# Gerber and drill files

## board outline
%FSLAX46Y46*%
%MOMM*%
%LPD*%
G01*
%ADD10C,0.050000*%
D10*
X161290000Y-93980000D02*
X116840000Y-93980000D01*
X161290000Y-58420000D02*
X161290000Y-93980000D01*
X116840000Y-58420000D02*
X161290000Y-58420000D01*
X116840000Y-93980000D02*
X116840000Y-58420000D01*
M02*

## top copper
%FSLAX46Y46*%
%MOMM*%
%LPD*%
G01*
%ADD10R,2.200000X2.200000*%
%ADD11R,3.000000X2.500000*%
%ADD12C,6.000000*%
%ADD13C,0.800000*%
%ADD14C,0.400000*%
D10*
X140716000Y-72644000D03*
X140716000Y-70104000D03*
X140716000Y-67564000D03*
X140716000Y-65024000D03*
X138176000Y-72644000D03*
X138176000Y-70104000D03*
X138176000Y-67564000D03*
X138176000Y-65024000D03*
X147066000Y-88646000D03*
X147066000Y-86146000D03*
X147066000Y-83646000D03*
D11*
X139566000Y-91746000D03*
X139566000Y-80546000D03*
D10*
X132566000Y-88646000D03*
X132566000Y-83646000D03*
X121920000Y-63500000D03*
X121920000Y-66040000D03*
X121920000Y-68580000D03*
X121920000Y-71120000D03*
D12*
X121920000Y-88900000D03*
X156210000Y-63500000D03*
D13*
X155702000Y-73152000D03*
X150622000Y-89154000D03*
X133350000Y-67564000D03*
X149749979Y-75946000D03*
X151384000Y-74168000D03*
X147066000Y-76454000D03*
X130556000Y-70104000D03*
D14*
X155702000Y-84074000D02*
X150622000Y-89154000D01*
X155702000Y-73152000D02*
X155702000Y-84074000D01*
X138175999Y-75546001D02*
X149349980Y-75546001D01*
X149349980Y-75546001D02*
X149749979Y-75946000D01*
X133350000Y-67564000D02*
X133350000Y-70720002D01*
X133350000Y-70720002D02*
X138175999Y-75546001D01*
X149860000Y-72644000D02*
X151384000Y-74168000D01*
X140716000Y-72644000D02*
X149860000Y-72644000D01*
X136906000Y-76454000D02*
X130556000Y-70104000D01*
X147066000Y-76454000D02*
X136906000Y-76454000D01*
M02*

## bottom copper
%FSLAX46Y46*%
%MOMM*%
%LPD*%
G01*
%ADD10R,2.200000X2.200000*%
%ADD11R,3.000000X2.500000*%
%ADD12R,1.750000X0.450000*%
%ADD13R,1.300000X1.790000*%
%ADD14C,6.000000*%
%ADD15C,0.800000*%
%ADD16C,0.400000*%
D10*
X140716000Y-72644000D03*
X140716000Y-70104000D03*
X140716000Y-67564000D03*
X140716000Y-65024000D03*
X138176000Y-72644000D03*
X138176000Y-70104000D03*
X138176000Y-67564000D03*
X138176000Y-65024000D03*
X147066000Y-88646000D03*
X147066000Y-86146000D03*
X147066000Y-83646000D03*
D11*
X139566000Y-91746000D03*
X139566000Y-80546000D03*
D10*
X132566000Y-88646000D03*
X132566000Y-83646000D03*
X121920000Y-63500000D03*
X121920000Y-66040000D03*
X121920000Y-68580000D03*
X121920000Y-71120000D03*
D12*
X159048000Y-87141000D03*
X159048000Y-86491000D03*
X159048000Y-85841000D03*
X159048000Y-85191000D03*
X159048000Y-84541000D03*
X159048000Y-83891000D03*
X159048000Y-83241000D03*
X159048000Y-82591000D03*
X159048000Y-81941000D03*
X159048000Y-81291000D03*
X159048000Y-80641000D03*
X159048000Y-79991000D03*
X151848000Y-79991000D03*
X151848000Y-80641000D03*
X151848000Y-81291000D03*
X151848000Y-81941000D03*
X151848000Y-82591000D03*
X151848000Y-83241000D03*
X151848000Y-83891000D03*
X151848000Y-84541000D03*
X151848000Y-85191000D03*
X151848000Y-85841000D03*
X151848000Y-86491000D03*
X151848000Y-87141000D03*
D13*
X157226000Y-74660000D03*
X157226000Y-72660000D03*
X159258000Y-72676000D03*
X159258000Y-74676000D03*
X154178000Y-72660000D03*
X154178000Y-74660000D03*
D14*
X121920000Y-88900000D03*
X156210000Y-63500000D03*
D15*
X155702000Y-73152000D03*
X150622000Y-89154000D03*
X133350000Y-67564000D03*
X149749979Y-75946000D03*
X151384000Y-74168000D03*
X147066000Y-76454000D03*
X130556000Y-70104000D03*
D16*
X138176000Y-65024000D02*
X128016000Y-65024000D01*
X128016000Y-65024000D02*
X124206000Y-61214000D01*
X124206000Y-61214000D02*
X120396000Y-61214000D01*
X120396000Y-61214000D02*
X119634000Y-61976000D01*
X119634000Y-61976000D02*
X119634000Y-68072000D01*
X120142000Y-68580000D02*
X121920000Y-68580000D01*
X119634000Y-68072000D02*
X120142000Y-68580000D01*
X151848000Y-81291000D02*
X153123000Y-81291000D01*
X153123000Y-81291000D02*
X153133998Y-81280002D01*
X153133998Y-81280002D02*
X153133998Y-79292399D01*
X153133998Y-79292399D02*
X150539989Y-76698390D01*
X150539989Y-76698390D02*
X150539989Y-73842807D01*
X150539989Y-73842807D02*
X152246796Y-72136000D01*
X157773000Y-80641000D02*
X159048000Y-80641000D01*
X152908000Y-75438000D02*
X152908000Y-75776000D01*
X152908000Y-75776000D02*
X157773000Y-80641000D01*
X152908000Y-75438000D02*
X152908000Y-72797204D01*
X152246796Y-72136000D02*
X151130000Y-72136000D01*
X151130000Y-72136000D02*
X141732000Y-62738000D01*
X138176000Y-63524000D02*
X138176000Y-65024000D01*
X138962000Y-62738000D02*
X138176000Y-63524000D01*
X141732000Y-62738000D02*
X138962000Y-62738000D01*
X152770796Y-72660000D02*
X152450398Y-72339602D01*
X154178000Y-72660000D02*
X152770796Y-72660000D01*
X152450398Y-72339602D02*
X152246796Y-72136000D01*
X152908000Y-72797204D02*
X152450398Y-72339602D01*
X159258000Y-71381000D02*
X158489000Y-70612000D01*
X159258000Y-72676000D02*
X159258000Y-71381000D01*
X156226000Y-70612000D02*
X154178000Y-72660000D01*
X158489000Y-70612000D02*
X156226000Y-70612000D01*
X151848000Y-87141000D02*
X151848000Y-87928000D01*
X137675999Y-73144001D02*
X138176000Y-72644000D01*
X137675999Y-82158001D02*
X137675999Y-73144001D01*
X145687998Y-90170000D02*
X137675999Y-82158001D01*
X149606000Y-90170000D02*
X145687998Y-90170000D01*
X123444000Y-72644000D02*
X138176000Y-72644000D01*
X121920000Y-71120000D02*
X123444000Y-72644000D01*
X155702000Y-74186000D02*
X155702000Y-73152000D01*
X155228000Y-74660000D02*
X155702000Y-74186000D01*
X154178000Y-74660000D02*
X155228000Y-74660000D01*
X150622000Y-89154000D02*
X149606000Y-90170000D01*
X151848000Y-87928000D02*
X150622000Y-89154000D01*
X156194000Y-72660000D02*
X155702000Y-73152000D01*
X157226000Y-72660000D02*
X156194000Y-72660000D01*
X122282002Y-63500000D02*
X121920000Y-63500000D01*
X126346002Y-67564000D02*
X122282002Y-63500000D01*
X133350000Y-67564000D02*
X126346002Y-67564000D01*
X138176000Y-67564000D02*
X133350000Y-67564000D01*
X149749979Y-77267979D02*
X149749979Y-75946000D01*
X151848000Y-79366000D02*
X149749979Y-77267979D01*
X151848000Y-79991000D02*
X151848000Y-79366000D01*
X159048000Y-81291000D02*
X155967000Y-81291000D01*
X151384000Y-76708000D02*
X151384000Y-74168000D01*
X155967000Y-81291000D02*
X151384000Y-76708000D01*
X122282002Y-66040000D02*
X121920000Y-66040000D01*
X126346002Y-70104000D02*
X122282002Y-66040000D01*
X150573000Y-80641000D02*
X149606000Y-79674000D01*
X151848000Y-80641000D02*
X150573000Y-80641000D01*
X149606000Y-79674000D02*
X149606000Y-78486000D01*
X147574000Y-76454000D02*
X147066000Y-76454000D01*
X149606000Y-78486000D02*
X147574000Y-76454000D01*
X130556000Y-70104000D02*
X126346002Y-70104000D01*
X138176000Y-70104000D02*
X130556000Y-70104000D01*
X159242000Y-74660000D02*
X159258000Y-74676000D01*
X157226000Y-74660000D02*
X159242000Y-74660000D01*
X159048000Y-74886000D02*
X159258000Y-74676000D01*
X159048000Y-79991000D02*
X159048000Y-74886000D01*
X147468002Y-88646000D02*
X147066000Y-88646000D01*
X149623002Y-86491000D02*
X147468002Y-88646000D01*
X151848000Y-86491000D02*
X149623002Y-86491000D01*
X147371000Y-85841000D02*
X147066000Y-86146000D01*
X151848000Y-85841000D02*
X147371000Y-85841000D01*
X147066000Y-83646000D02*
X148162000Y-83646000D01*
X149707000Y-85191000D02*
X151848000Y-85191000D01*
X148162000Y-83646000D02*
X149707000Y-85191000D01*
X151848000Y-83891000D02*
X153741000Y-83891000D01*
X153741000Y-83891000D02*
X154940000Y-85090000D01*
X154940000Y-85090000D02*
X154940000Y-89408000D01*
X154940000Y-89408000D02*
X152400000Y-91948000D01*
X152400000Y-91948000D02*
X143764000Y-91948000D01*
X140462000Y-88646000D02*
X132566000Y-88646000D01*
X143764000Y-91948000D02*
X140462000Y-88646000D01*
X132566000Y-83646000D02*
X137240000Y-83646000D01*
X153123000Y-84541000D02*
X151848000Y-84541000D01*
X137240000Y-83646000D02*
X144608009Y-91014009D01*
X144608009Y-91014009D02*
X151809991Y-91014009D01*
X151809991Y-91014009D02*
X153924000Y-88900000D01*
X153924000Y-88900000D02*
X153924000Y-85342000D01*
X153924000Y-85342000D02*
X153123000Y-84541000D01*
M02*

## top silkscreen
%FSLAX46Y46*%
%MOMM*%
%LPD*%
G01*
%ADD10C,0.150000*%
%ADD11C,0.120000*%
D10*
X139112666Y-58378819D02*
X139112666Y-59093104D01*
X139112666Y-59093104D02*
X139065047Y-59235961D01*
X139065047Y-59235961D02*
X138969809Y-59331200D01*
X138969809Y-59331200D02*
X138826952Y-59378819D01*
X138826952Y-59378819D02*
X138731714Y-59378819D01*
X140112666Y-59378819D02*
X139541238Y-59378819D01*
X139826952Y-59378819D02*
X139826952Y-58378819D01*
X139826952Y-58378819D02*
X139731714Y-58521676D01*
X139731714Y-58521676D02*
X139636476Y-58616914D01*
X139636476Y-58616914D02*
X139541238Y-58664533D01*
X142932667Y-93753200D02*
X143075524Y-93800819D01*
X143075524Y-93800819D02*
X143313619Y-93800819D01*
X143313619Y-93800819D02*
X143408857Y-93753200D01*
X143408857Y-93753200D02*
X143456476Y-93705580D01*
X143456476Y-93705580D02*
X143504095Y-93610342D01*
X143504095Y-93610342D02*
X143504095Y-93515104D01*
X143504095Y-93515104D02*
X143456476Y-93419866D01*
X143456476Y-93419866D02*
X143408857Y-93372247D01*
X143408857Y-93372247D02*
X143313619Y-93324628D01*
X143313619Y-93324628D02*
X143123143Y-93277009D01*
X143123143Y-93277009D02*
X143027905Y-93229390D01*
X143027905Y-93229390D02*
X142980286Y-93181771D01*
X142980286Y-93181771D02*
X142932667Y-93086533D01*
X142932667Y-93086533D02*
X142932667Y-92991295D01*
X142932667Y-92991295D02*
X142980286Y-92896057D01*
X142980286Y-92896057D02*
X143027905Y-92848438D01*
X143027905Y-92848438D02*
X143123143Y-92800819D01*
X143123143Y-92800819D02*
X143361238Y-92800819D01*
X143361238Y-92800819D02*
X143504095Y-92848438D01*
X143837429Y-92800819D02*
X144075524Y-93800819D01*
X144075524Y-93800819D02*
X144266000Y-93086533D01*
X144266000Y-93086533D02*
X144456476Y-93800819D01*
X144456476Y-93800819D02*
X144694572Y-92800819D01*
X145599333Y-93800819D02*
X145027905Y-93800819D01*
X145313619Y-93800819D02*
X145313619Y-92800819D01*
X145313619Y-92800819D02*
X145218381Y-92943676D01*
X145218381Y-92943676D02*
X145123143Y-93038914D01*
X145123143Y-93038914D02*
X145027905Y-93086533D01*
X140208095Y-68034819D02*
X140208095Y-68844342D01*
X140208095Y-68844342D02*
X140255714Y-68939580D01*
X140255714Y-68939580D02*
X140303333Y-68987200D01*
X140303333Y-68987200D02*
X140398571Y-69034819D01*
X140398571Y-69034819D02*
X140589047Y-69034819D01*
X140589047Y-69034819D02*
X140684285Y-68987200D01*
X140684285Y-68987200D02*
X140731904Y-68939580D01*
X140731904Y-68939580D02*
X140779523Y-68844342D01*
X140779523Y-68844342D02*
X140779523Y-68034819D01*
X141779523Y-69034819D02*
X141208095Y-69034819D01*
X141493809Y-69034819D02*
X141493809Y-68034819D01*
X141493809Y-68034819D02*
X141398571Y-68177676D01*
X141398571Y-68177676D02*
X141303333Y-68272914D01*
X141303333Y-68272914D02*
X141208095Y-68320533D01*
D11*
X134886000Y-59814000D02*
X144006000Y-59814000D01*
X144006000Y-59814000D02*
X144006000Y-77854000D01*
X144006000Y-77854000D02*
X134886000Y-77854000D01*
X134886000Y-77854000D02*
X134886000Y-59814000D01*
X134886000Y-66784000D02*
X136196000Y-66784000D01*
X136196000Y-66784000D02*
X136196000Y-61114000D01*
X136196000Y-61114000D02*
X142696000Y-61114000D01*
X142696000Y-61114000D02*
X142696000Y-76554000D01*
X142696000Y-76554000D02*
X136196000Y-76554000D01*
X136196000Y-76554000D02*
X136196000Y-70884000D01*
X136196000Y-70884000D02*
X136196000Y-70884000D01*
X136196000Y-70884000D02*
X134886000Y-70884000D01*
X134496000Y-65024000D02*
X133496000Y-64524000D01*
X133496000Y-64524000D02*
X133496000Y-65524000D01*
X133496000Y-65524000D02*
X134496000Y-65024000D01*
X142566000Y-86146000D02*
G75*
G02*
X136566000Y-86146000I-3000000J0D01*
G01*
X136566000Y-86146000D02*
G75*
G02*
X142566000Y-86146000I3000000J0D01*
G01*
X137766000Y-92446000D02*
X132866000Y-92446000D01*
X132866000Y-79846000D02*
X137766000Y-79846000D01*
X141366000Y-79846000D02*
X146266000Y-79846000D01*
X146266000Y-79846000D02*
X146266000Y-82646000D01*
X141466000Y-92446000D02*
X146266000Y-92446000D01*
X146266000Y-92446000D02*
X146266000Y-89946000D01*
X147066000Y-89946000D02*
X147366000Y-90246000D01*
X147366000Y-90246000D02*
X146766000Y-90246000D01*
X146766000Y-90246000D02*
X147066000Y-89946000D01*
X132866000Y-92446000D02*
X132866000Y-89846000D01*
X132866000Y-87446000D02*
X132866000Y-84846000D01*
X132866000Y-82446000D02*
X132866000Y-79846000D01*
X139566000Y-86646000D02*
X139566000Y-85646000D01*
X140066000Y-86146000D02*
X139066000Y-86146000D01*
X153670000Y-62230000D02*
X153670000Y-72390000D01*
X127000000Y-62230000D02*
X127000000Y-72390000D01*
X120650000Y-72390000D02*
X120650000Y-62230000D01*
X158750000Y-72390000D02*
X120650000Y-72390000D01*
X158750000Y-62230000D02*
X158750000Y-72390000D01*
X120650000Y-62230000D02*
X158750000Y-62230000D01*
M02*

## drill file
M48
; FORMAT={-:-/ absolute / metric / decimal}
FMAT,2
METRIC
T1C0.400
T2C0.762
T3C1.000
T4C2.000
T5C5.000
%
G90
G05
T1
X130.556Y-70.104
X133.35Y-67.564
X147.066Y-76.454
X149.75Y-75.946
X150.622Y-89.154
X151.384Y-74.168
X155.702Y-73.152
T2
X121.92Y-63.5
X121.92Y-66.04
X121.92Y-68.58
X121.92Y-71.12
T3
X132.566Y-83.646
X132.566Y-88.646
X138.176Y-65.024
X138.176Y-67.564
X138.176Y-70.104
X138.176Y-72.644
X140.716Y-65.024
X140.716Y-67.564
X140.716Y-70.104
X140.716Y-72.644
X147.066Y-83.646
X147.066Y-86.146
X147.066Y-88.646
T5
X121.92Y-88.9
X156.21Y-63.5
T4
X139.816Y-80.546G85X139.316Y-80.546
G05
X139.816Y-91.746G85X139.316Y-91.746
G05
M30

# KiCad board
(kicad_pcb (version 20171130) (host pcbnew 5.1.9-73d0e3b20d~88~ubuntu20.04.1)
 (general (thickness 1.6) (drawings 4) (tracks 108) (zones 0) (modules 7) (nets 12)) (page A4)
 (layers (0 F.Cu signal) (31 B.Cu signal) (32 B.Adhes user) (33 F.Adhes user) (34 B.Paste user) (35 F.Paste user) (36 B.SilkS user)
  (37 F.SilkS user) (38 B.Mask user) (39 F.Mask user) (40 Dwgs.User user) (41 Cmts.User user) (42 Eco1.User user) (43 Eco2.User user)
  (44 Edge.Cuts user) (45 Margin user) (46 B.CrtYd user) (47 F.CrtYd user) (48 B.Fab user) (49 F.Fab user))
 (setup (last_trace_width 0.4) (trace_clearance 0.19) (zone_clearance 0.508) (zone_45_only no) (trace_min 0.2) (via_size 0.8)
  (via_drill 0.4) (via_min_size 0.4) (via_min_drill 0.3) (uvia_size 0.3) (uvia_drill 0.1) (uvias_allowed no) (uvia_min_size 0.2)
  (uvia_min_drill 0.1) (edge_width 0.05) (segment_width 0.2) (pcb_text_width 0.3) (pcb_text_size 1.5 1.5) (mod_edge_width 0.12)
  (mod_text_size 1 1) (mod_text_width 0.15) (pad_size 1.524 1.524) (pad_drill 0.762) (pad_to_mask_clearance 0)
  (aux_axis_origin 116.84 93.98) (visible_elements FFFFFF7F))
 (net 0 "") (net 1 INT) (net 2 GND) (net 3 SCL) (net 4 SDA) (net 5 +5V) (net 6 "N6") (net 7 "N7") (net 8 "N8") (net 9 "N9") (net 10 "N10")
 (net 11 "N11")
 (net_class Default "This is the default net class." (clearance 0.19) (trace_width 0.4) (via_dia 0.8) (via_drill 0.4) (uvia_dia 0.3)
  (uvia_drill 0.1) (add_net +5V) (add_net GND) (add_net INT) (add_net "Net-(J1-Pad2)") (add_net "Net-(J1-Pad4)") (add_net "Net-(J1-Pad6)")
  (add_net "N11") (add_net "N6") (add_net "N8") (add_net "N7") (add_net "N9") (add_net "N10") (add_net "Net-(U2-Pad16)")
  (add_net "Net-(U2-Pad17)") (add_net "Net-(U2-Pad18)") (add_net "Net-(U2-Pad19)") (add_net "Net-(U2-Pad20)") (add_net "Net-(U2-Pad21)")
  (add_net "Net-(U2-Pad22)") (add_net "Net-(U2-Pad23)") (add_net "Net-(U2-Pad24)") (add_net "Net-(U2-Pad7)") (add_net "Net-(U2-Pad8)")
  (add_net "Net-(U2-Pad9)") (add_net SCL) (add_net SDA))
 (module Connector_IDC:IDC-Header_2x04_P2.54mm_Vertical (layer F.Cu) (at 138.176 65.024)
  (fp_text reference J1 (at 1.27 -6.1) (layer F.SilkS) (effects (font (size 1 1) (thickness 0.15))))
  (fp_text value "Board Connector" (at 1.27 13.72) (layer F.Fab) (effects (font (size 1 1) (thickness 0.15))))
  (fp_line (start -3.29 -5.21) (end 5.83 -5.21) (layer F.SilkS) (width 0.12))
  (fp_line (start 5.83 -5.21) (end 5.83 12.83) (layer F.SilkS) (width 0.12))
  (fp_line (start 5.83 12.83) (end -3.29 12.83) (layer F.SilkS) (width 0.12))
  (fp_line (start -3.29 12.83) (end -3.29 -5.21) (layer F.SilkS) (width 0.12))
  (fp_line (start -3.29 1.76) (end -1.98 1.76) (layer F.SilkS) (width 0.12))
  (fp_line (start -1.98 1.76) (end -1.98 -3.91) (layer F.SilkS) (width 0.12))
  (fp_line (start -1.98 -3.91) (end 4.52 -3.91) (layer F.SilkS) (width 0.12))
  (fp_line (start 4.52 -3.91) (end 4.52 11.53) (layer F.SilkS) (width 0.12))
  (fp_line (start 4.52 11.53) (end -1.98 11.53) (layer F.SilkS) (width 0.12))
  (fp_line (start -1.98 11.53) (end -1.98 5.86) (layer F.SilkS) (width 0.12))
  (fp_line (start -1.98 5.86) (end -1.98 5.86) (layer F.SilkS) (width 0.12))
  (fp_line (start -1.98 5.86) (end -3.29 5.86) (layer F.SilkS) (width 0.12))
  (fp_line (start -3.68 0) (end -4.68 -0.5) (layer F.SilkS) (width 0.12))
  (fp_line (start -4.68 -0.5) (end -4.68 0.5) (layer F.SilkS) (width 0.12))
  (fp_line (start -4.68 0.5) (end -3.68 0) (layer F.SilkS) (width 0.12))
  (pad 8 thru_hole rect (at 2.54 7.62) (size 2.2 2.2) (drill 1) (layers *.Cu *.Mask) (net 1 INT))
  (pad 6 thru_hole rect (at 2.54 5.08) (size 2.2 2.2) (drill 1) (layers *.Cu *.Mask))
  (pad 4 thru_hole rect (at 2.54 2.54) (size 2.2 2.2) (drill 1) (layers *.Cu *.Mask))
  (pad 2 thru_hole rect (at 2.54 0) (size 2.2 2.2) (drill 1) (layers *.Cu *.Mask))
  (pad 7 thru_hole rect (at 0 7.62) (size 2.2 2.2) (drill 1) (layers *.Cu *.Mask) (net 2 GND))
  (pad 5 thru_hole rect (at 0 5.08) (size 2.2 2.2) (drill 1) (layers *.Cu *.Mask) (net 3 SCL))
  (pad 3 thru_hole rect (at 0 2.54) (size 2.2 2.2) (drill 1) (layers *.Cu *.Mask) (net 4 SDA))
  (pad 1 thru_hole rect (at 0 0) (size 2.2 2.2) (drill 1) (layers *.Cu *.Mask) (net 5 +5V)))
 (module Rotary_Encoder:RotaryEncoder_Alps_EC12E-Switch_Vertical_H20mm (layer F.Cu) (at 147.066 88.646 180)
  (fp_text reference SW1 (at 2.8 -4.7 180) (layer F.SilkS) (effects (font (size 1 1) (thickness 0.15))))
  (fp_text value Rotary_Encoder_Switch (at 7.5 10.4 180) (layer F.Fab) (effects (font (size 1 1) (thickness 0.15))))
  (fp_circle (center 7.5 2.5) (end 10.5 2.5) (layer F.SilkS) (width 0.12))
  (fp_line (start 9.3 -3.8) (end 14.2 -3.8) (layer F.SilkS) (width 0.12))
  (fp_line (start 14.2 8.8) (end 9.3 8.8) (layer F.SilkS) (width 0.12))
  (fp_line (start 5.7 8.8) (end 0.8 8.8) (layer F.SilkS) (width 0.12))
  (fp_line (start 0.8 8.8) (end 0.8 6) (layer F.SilkS) (width 0.12))
  (fp_line (start 5.6 -3.8) (end 0.8 -3.8) (layer F.SilkS) (width 0.12))
  (fp_line (start 0.8 -3.8) (end 0.8 -1.3) (layer F.SilkS) (width 0.12))
  (fp_line (start 0 -1.3) (end -0.3 -1.6) (layer F.SilkS) (width 0.12))
  (fp_line (start -0.3 -1.6) (end 0.3 -1.6) (layer F.SilkS) (width 0.12))
  (fp_line (start 0.3 -1.6) (end 0 -1.3) (layer F.SilkS) (width 0.12))
  (fp_line (start 14.2 -3.8) (end 14.2 -1.2) (layer F.SilkS) (width 0.12))
  (fp_line (start 14.2 1.2) (end 14.2 3.8) (layer F.SilkS) (width 0.12))
  (fp_line (start 14.2 6.2) (end 14.2 8.8) (layer F.SilkS) (width 0.12))
  (fp_line (start 7.5 2) (end 7.5 3) (layer F.SilkS) (width 0.12))
  (fp_line (start 7 2.5) (end 8 2.5) (layer F.SilkS) (width 0.12))
  (pad A thru_hole rect (at 0 0 180) (size 2.2 2.2) (drill 1) (layers *.Cu *.Mask) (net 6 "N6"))
  (pad C thru_hole rect (at 0 2.5 180) (size 2.2 2.2) (drill 1) (layers *.Cu *.Mask) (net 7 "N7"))
  (pad B thru_hole rect (at 0 5 180) (size 2.2 2.2) (drill 1) (layers *.Cu *.Mask) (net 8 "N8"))
  (pad MP thru_hole rect (at 7.5 -3.1 180) (size 3 2.5) (drill oval 2.5 2) (layers *.Cu *.Mask))
  (pad MP thru_hole rect (at 7.5 8.1 180) (size 3 2.5) (drill oval 2.5 2) (layers *.Cu *.Mask))
  (pad S1 thru_hole rect (at 14.5 0 180) (size 2.2 2.2) (drill 1) (layers *.Cu *.Mask) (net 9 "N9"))
  (pad S2 thru_hole rect (at 14.5 5 180) (size 2.2 2.2) (drill 1) (layers *.Cu *.Mask) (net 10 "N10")))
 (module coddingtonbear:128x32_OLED (layer F.Cu) (at 129.54 68.58)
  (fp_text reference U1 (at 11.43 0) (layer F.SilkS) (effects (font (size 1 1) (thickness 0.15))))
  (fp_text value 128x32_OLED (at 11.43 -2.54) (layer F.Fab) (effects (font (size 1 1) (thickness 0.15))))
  (fp_line (start 24.13 -6.35) (end 24.13 3.81) (layer F.SilkS) (width 0.12))
  (fp_line (start -2.54 -6.35) (end -2.54 3.81) (layer F.SilkS) (width 0.12))
  (fp_line (start -8.89 3.81) (end -8.89 -6.35) (layer F.SilkS) (width 0.12))
  (fp_line (start 29.21 3.81) (end -8.89 3.81) (layer F.SilkS) (width 0.12))
  (fp_line (start 29.21 -6.35) (end 29.21 3.81) (layer F.SilkS) (width 0.12))
  (fp_line (start -8.89 -6.35) (end 29.21 -6.35) (layer F.SilkS) (width 0.12))
  (pad 4 thru_hole rect (at -7.62 -5.08) (size 2.2 2.2) (drill 0.762) (layers *.Cu *.Mask) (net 4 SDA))
  (pad 3 thru_hole rect (at -7.62 -2.54) (size 2.2 2.2) (drill 0.762) (layers *.Cu *.Mask) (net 3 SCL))
  (pad 2 thru_hole rect (at -7.62 0) (size 2.2 2.2) (drill 0.762) (layers *.Cu *.Mask) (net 5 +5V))
  (pad 1 thru_hole rect (at -7.62 2.54) (size 2.2 2.2) (drill 0.762) (layers *.Cu *.Mask) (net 2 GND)))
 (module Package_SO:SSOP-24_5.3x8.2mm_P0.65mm (layer B.Cu) (at 155.448 83.566)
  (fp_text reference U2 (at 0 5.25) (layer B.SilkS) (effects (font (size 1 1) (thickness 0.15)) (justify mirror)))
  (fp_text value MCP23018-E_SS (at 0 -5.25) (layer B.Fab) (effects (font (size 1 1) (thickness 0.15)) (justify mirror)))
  (pad 24 smd rect (at 3.6 3.575) (size 1.75 0.45) (layers B.Cu B.Paste B.Mask))
  (pad 23 smd rect (at 3.6 2.925) (size 1.75 0.45) (layers B.Cu B.Paste B.Mask))
  (pad 22 smd rect (at 3.6 2.275) (size 1.75 0.45) (layers B.Cu B.Paste B.Mask))
  (pad 21 smd rect (at 3.6 1.625) (size 1.75 0.45) (layers B.Cu B.Paste B.Mask))
  (pad 20 smd rect (at 3.6 0.975) (size 1.75 0.45) (layers B.Cu B.Paste B.Mask))
  (pad 19 smd rect (at 3.6 0.325) (size 1.75 0.45) (layers B.Cu B.Paste B.Mask))
  (pad 18 smd rect (at 3.6 -0.325) (size 1.75 0.45) (layers B.Cu B.Paste B.Mask))
  (pad 17 smd rect (at 3.6 -0.975) (size 1.75 0.45) (layers B.Cu B.Paste B.Mask))
  (pad 16 smd rect (at 3.6 -1.625) (size 1.75 0.45) (layers B.Cu B.Paste B.Mask))
  (pad 15 smd rect (at 3.6 -2.275) (size 1.75 0.45) (layers B.Cu B.Paste B.Mask) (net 1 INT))
  (pad 14 smd rect (at 3.6 -2.925) (size 1.75 0.45) (layers B.Cu B.Paste B.Mask) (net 5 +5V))
  (pad 13 smd rect (at 3.6 -3.575) (size 1.75 0.45) (layers B.Cu B.Paste B.Mask) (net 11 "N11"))
  (pad 12 smd rect (at -3.6 -3.575) (size 1.75 0.45) (layers B.Cu B.Paste B.Mask) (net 4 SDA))
  (pad 11 smd rect (at -3.6 -2.925) (size 1.75 0.45) (layers B.Cu B.Paste B.Mask) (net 3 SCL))
  (pad 10 smd rect (at -3.6 -2.275) (size 1.75 0.45) (layers B.Cu B.Paste B.Mask) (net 5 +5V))
  (pad 9 smd rect (at -3.6 -1.625) (size 1.75 0.45) (layers B.Cu B.Paste B.Mask))
  (pad 8 smd rect (at -3.6 -0.975) (size 1.75 0.45) (layers B.Cu B.Paste B.Mask))
  (pad 7 smd rect (at -3.6 -0.325) (size 1.75 0.45) (layers B.Cu B.Paste B.Mask))
  (pad 6 smd rect (at -3.6 0.325) (size 1.75 0.45) (layers B.Cu B.Paste B.Mask) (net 9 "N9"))
  (pad 5 smd rect (at -3.6 0.975) (size 1.75 0.45) (layers B.Cu B.Paste B.Mask) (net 10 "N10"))
  (pad 4 smd rect (at -3.6 1.625) (size 1.75 0.45) (layers B.Cu B.Paste B.Mask) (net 8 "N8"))
  (pad 3 smd rect (at -3.6 2.275) (size 1.75 0.45) (layers B.Cu B.Paste B.Mask) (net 7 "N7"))
  (pad 2 smd rect (at -3.6 2.925) (size 1.75 0.45) (layers B.Cu B.Paste B.Mask) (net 6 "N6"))
  (pad 1 smd rect (at -3.6 3.575) (size 1.75 0.45) (layers B.Cu B.Paste B.Mask) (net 2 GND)))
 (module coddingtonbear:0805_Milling (layer B.Cu) (at 157.226 73.66 90)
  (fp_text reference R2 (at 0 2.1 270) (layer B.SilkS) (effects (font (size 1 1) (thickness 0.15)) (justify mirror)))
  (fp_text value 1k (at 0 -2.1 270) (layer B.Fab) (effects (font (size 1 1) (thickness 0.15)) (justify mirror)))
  (pad 1 smd rect (at -1 0 90) (size 1.79 1.3) (layers B.Cu B.Paste B.Mask) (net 11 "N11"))
  (pad 2 smd rect (at 1 0 90) (size 1.79 1.3) (layers B.Cu B.Paste B.Mask) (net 2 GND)))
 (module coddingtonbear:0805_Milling (layer B.Cu) (at 159.258 73.676 270)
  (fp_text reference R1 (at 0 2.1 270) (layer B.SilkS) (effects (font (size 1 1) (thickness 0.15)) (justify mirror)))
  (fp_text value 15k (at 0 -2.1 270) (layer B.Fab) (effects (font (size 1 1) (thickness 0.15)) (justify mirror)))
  (pad 1 smd rect (at -1 0 270) (size 1.79 1.3) (layers B.Cu B.Paste B.Mask) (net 5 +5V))
  (pad 2 smd rect (at 1 0 270) (size 1.79 1.3) (layers B.Cu B.Paste B.Mask) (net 11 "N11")))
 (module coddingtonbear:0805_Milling (layer B.Cu) (at 154.178 73.66 270)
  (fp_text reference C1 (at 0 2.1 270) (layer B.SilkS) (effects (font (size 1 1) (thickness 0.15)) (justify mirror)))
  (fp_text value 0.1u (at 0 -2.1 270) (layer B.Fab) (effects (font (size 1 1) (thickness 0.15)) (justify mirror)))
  (pad 1 smd rect (at -1 0 270) (size 1.79 1.3) (layers B.Cu B.Paste B.Mask) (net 5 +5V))
  (pad 2 smd rect (at 1 0 270) (size 1.79 1.3) (layers B.Cu B.Paste B.Mask) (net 2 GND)))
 (gr_line (start 161.29 93.98) (end 116.84 93.98) (layer Edge.Cuts) (width 0.05))
 (gr_line (start 161.29 58.42) (end 161.29 93.98) (layer Edge.Cuts) (width 0.05))
 (gr_line (start 116.84 58.42) (end 161.29 58.42) (layer Edge.Cuts) (width 0.05))
 (gr_line (start 116.84 93.98) (end 116.84 58.42) (layer Edge.Cuts) (width 0.05))
 (via (at 121.92 88.9) (size 6) (drill 5) (layers F.Cu B.Cu) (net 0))
 (via (at 156.21 63.5) (size 6) (drill 5) (layers F.Cu B.Cu) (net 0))
 (segment (start 138.176 65.024) (end 128.016 65.024) (width 0.4) (layer B.Cu) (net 5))
 (segment (start 128.016 65.024) (end 124.206 61.214) (width 0.4) (layer B.Cu) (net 5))
 (segment (start 124.206 61.214) (end 120.396 61.214) (width 0.4) (layer B.Cu) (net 5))
 (segment (start 120.396 61.214) (end 119.634 61.976) (width 0.4) (layer B.Cu) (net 5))
 (segment (start 119.634 61.976) (end 119.634 68.072) (width 0.4) (layer B.Cu) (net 5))
 (segment (start 120.142 68.58) (end 121.92 68.58) (width 0.4) (layer B.Cu) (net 5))
 (segment (start 119.634 68.072) (end 120.142 68.58) (width 0.4) (layer B.Cu) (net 5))
 (segment (start 151.848 81.291) (end 153.123 81.291) (width 0.4) (layer B.Cu) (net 5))
 (segment (start 153.123 81.291) (end 153.133998 81.280002) (width 0.4) (layer B.Cu) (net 5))
 (segment (start 153.133998 81.280002) (end 153.133998 79.292399) (width 0.4) (layer B.Cu) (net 5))
 (segment (start 153.133998 79.292399) (end 150.539989 76.69839) (width 0.4) (layer B.Cu) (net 5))
 (segment (start 150.539989 76.69839) (end 150.539989 73.842807) (width 0.4) (layer B.Cu) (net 5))
 (segment (start 150.539989 73.842807) (end 152.246796 72.136) (width 0.4) (layer B.Cu) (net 5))
 (segment (start 157.773 80.641) (end 159.048 80.641) (width 0.4) (layer B.Cu) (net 5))
 (segment (start 152.908 75.438) (end 152.908 75.776) (width 0.4) (layer B.Cu) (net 5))
 (segment (start 152.908 75.776) (end 157.773 80.641) (width 0.4) (layer B.Cu) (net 5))
 (segment (start 152.908 75.438) (end 152.908 72.797204) (width 0.4) (layer B.Cu) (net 5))
 (segment (start 152.246796 72.136) (end 151.13 72.136) (width 0.4) (layer B.Cu) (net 5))
 (segment (start 151.13 72.136) (end 141.732 62.738) (width 0.4) (layer B.Cu) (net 5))
 (segment (start 138.176 63.524) (end 138.176 65.024) (width 0.4) (layer B.Cu) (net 5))
 (segment (start 138.962 62.738) (end 138.176 63.524) (width 0.4) (layer B.Cu) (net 5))
 (segment (start 141.732 62.738) (end 138.962 62.738) (width 0.4) (layer B.Cu) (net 5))
 (segment (start 152.770796 72.66) (end 152.450398 72.339602) (width 0.4) (layer B.Cu) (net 5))
 (segment (start 154.178 72.66) (end 152.770796 72.66) (width 0.4) (layer B.Cu) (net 5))
 (segment (start 152.450398 72.339602) (end 152.246796 72.136) (width 0.4) (layer B.Cu) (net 5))
 (segment (start 152.908 72.797204) (end 152.450398 72.339602) (width 0.4) (layer B.Cu) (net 5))
 (segment (start 159.258 71.381) (end 158.489 70.612) (width 0.4) (layer B.Cu) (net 5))
 (segment (start 159.258 72.676) (end 159.258 71.381) (width 0.4) (layer B.Cu) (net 5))
 (segment (start 156.226 70.612) (end 154.178 72.66) (width 0.4) (layer B.Cu) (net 5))
 (segment (start 158.489 70.612) (end 156.226 70.612) (width 0.4) (layer B.Cu) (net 5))
 (segment (start 151.848 87.141) (end 151.848 87.928) (width 0.4) (layer B.Cu) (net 2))
 (segment (start 137.675999 73.144001) (end 138.176 72.644) (width 0.4) (layer B.Cu) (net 2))
 (segment (start 137.675999 82.158001) (end 137.675999 73.144001) (width 0.4) (layer B.Cu) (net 2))
 (segment (start 145.687998 90.17) (end 137.675999 82.158001) (width 0.4) (layer B.Cu) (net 2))
 (segment (start 149.606 90.17) (end 145.687998 90.17) (width 0.4) (layer B.Cu) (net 2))
 (segment (start 123.444 72.644) (end 138.176 72.644) (width 0.4) (layer B.Cu) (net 2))
 (segment (start 121.92 71.12) (end 123.444 72.644) (width 0.4) (layer B.Cu) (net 2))
 (via (at 155.702 73.152) (size 0.8) (drill 0.4) (layers F.Cu B.Cu) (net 2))
 (segment (start 155.702 74.186) (end 155.702 73.152) (width 0.4) (layer B.Cu) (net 2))
 (segment (start 155.228 74.66) (end 155.702 74.186) (width 0.4) (layer B.Cu) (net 2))
 (segment (start 154.178 74.66) (end 155.228 74.66) (width 0.4) (layer B.Cu) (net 2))
 (segment (start 155.702 84.074) (end 150.622 89.154) (width 0.4) (layer F.Cu) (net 2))
 (via (at 150.622 89.154) (size 0.8) (drill 0.4) (layers F.Cu B.Cu) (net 2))
 (segment (start 155.702 73.152) (end 155.702 84.074) (width 0.4) (layer F.Cu) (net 2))
 (segment (start 150.622 89.154) (end 149.606 90.17) (width 0.4) (layer B.Cu) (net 2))
 (segment (start 151.848 87.928) (end 150.622 89.154) (width 0.4) (layer B.Cu) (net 2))
 (segment (start 156.194 72.66) (end 155.702 73.152) (width 0.4) (layer B.Cu) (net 2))
 (segment (start 157.226 72.66) (end 156.194 72.66) (width 0.4) (layer B.Cu) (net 2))
 (segment (start 122.282002 63.5) (end 121.92 63.5) (width 0.4) (layer B.Cu) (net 4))
 (segment (start 126.346002 67.564) (end 122.282002 63.5) (width 0.4) (layer B.Cu) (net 4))
 (via (at 133.35 67.564) (size 0.8) (drill 0.4) (layers F.Cu B.Cu) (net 4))
 (segment (start 133.35 67.564) (end 126.346002 67.564) (width 0.4) (layer B.Cu) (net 4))
 (segment (start 138.176 67.564) (end 133.35 67.564) (width 0.4) (layer B.Cu) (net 4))
 (segment (start 138.175999 75.546001) (end 149.34998 75.546001) (width 0.4) (layer F.Cu) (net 4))
 (segment (start 149.34998 75.546001) (end 149.749979 75.946) (width 0.4) (layer F.Cu) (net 4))
 (segment (start 149.749979 77.267979) (end 149.749979 75.946) (width 0.4) (layer B.Cu) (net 4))
 (via (at 149.749979 75.946) (size 0.8) (drill 0.4) (layers F.Cu B.Cu) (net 4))
 (segment (start 151.848 79.366) (end 149.749979 77.267979) (width 0.4) (layer B.Cu) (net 4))
 (segment (start 133.35 67.564) (end 133.35 70.720002) (width 0.4) (layer F.Cu) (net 4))
 (segment (start 133.35 70.720002) (end 138.175999 75.546001) (width 0.4) (layer F.Cu) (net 4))
 (segment (start 151.848 79.991) (end 151.848 79.366) (width 0.4) (layer B.Cu) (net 4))
 (segment (start 159.048 81.291) (end 155.967 81.291) (width 0.4) (layer B.Cu) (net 1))
 (segment (start 149.86 72.644) (end 151.384 74.168) (width 0.4) (layer F.Cu) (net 1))
 (segment (start 140.716 72.644) (end 149.86 72.644) (width 0.4) (layer F.Cu) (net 1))
 (segment (start 151.384 76.708) (end 151.384 74.168) (width 0.4) (layer B.Cu) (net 1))
 (via (at 151.384 74.168) (size 0.8) (drill 0.4) (layers F.Cu B.Cu) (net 1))
 (segment (start 155.967 81.291) (end 151.384 76.708) (width 0.4) (layer B.Cu) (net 1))
 (segment (start 122.282002 66.04) (end 121.92 66.04) (width 0.4) (layer B.Cu) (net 3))
 (segment (start 126.346002 70.104) (end 122.282002 66.04) (width 0.4) (layer B.Cu) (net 3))
 (segment (start 150.573 80.641) (end 149.606 79.674) (width 0.4) (layer B.Cu) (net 3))
 (segment (start 151.848 80.641) (end 150.573 80.641) (width 0.4) (layer B.Cu) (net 3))
 (segment (start 149.606 79.674) (end 149.606 78.486) (width 0.4) (layer B.Cu) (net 3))
 (segment (start 147.574 76.454) (end 147.066 76.454) (width 0.4) (layer B.Cu) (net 3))
 (via (at 147.066 76.454) (size 0.8) (drill 0.4) (layers F.Cu B.Cu) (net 3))
 (segment (start 149.606 78.486) (end 147.574 76.454) (width 0.4) (layer B.Cu) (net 3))
 (via (at 130.556 70.104) (size 0.8) (drill 0.4) (layers F.Cu B.Cu) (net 3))
 (segment (start 136.906 76.454) (end 130.556 70.104) (width 0.4) (layer F.Cu) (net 3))
 (segment (start 147.066 76.454) (end 136.906 76.454) (width 0.4) (layer F.Cu) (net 3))
 (segment (start 130.556 70.104) (end 126.346002 70.104) (width 0.4) (layer B.Cu) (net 3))
 (segment (start 138.176 70.104) (end 130.556 70.104) (width 0.4) (layer B.Cu) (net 3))
 (segment (start 159.242 74.66) (end 159.258 74.676) (width 0.4) (layer B.Cu) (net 11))
 (segment (start 157.226 74.66) (end 159.242 74.66) (width 0.4) (layer B.Cu) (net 11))
 (segment (start 159.048 74.886) (end 159.258 74.676) (width 0.4) (layer B.Cu) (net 11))
 (segment (start 159.048 79.991) (end 159.048 74.886) (width 0.4) (layer B.Cu) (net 11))
 (segment (start 147.468002 88.646) (end 147.066 88.646) (width 0.4) (layer B.Cu) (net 6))
 (segment (start 149.623002 86.491) (end 147.468002 88.646) (width 0.4) (layer B.Cu) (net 6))
 (segment (start 151.848 86.491) (end 149.623002 86.491) (width 0.4) (layer B.Cu) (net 6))
 (segment (start 147.371 85.841) (end 147.066 86.146) (width 0.4) (layer B.Cu) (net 7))
 (segment (start 151.848 85.841) (end 147.371 85.841) (width 0.4) (layer B.Cu) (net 7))
 (segment (start 147.066 83.646) (end 148.162 83.646) (width 0.4) (layer B.Cu) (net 8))
 (segment (start 149.707 85.191) (end 151.848 85.191) (width 0.4) (layer B.Cu) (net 8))
 (segment (start 148.162 83.646) (end 149.707 85.191) (width 0.4) (layer B.Cu) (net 8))
 (segment (start 151.848 83.891) (end 153.741 83.891) (width 0.4) (layer B.Cu) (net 9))
 (segment (start 153.741 83.891) (end 154.94 85.09) (width 0.4) (layer B.Cu) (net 9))
 (segment (start 154.94 85.09) (end 154.94 89.408) (width 0.4) (layer B.Cu) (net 9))
 (segment (start 154.94 89.408) (end 152.4 91.948) (width 0.4) (layer B.Cu) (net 9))
 (segment (start 152.4 91.948) (end 143.764 91.948) (width 0.4) (layer B.Cu) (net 9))
 (segment (start 140.462 88.646) (end 132.566 88.646) (width 0.4) (layer B.Cu) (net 9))
 (segment (start 143.764 91.948) (end 140.462 88.646) (width 0.4) (layer B.Cu) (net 9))
 (segment (start 132.566 83.646) (end 137.24 83.646) (width 0.4) (layer B.Cu) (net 10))
 (segment (start 153.123 84.541) (end 151.848 84.541) (width 0.4) (layer B.Cu) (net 10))
 (segment (start 137.24 83.646) (end 144.608009 91.014009) (width 0.4) (layer B.Cu) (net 10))
 (segment (start 144.608009 91.014009) (end 151.809991 91.014009) (width 0.4) (layer B.Cu) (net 10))
 (segment (start 151.809991 91.014009) (end 153.924 88.9) (width 0.4) (layer B.Cu) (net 10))
 (segment (start 153.924 88.9) (end 153.924 85.342) (width 0.4) (layer B.Cu) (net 10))
 (segment (start 153.924 85.342) (end 153.123 84.541) (width 0.4) (layer B.Cu) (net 10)))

